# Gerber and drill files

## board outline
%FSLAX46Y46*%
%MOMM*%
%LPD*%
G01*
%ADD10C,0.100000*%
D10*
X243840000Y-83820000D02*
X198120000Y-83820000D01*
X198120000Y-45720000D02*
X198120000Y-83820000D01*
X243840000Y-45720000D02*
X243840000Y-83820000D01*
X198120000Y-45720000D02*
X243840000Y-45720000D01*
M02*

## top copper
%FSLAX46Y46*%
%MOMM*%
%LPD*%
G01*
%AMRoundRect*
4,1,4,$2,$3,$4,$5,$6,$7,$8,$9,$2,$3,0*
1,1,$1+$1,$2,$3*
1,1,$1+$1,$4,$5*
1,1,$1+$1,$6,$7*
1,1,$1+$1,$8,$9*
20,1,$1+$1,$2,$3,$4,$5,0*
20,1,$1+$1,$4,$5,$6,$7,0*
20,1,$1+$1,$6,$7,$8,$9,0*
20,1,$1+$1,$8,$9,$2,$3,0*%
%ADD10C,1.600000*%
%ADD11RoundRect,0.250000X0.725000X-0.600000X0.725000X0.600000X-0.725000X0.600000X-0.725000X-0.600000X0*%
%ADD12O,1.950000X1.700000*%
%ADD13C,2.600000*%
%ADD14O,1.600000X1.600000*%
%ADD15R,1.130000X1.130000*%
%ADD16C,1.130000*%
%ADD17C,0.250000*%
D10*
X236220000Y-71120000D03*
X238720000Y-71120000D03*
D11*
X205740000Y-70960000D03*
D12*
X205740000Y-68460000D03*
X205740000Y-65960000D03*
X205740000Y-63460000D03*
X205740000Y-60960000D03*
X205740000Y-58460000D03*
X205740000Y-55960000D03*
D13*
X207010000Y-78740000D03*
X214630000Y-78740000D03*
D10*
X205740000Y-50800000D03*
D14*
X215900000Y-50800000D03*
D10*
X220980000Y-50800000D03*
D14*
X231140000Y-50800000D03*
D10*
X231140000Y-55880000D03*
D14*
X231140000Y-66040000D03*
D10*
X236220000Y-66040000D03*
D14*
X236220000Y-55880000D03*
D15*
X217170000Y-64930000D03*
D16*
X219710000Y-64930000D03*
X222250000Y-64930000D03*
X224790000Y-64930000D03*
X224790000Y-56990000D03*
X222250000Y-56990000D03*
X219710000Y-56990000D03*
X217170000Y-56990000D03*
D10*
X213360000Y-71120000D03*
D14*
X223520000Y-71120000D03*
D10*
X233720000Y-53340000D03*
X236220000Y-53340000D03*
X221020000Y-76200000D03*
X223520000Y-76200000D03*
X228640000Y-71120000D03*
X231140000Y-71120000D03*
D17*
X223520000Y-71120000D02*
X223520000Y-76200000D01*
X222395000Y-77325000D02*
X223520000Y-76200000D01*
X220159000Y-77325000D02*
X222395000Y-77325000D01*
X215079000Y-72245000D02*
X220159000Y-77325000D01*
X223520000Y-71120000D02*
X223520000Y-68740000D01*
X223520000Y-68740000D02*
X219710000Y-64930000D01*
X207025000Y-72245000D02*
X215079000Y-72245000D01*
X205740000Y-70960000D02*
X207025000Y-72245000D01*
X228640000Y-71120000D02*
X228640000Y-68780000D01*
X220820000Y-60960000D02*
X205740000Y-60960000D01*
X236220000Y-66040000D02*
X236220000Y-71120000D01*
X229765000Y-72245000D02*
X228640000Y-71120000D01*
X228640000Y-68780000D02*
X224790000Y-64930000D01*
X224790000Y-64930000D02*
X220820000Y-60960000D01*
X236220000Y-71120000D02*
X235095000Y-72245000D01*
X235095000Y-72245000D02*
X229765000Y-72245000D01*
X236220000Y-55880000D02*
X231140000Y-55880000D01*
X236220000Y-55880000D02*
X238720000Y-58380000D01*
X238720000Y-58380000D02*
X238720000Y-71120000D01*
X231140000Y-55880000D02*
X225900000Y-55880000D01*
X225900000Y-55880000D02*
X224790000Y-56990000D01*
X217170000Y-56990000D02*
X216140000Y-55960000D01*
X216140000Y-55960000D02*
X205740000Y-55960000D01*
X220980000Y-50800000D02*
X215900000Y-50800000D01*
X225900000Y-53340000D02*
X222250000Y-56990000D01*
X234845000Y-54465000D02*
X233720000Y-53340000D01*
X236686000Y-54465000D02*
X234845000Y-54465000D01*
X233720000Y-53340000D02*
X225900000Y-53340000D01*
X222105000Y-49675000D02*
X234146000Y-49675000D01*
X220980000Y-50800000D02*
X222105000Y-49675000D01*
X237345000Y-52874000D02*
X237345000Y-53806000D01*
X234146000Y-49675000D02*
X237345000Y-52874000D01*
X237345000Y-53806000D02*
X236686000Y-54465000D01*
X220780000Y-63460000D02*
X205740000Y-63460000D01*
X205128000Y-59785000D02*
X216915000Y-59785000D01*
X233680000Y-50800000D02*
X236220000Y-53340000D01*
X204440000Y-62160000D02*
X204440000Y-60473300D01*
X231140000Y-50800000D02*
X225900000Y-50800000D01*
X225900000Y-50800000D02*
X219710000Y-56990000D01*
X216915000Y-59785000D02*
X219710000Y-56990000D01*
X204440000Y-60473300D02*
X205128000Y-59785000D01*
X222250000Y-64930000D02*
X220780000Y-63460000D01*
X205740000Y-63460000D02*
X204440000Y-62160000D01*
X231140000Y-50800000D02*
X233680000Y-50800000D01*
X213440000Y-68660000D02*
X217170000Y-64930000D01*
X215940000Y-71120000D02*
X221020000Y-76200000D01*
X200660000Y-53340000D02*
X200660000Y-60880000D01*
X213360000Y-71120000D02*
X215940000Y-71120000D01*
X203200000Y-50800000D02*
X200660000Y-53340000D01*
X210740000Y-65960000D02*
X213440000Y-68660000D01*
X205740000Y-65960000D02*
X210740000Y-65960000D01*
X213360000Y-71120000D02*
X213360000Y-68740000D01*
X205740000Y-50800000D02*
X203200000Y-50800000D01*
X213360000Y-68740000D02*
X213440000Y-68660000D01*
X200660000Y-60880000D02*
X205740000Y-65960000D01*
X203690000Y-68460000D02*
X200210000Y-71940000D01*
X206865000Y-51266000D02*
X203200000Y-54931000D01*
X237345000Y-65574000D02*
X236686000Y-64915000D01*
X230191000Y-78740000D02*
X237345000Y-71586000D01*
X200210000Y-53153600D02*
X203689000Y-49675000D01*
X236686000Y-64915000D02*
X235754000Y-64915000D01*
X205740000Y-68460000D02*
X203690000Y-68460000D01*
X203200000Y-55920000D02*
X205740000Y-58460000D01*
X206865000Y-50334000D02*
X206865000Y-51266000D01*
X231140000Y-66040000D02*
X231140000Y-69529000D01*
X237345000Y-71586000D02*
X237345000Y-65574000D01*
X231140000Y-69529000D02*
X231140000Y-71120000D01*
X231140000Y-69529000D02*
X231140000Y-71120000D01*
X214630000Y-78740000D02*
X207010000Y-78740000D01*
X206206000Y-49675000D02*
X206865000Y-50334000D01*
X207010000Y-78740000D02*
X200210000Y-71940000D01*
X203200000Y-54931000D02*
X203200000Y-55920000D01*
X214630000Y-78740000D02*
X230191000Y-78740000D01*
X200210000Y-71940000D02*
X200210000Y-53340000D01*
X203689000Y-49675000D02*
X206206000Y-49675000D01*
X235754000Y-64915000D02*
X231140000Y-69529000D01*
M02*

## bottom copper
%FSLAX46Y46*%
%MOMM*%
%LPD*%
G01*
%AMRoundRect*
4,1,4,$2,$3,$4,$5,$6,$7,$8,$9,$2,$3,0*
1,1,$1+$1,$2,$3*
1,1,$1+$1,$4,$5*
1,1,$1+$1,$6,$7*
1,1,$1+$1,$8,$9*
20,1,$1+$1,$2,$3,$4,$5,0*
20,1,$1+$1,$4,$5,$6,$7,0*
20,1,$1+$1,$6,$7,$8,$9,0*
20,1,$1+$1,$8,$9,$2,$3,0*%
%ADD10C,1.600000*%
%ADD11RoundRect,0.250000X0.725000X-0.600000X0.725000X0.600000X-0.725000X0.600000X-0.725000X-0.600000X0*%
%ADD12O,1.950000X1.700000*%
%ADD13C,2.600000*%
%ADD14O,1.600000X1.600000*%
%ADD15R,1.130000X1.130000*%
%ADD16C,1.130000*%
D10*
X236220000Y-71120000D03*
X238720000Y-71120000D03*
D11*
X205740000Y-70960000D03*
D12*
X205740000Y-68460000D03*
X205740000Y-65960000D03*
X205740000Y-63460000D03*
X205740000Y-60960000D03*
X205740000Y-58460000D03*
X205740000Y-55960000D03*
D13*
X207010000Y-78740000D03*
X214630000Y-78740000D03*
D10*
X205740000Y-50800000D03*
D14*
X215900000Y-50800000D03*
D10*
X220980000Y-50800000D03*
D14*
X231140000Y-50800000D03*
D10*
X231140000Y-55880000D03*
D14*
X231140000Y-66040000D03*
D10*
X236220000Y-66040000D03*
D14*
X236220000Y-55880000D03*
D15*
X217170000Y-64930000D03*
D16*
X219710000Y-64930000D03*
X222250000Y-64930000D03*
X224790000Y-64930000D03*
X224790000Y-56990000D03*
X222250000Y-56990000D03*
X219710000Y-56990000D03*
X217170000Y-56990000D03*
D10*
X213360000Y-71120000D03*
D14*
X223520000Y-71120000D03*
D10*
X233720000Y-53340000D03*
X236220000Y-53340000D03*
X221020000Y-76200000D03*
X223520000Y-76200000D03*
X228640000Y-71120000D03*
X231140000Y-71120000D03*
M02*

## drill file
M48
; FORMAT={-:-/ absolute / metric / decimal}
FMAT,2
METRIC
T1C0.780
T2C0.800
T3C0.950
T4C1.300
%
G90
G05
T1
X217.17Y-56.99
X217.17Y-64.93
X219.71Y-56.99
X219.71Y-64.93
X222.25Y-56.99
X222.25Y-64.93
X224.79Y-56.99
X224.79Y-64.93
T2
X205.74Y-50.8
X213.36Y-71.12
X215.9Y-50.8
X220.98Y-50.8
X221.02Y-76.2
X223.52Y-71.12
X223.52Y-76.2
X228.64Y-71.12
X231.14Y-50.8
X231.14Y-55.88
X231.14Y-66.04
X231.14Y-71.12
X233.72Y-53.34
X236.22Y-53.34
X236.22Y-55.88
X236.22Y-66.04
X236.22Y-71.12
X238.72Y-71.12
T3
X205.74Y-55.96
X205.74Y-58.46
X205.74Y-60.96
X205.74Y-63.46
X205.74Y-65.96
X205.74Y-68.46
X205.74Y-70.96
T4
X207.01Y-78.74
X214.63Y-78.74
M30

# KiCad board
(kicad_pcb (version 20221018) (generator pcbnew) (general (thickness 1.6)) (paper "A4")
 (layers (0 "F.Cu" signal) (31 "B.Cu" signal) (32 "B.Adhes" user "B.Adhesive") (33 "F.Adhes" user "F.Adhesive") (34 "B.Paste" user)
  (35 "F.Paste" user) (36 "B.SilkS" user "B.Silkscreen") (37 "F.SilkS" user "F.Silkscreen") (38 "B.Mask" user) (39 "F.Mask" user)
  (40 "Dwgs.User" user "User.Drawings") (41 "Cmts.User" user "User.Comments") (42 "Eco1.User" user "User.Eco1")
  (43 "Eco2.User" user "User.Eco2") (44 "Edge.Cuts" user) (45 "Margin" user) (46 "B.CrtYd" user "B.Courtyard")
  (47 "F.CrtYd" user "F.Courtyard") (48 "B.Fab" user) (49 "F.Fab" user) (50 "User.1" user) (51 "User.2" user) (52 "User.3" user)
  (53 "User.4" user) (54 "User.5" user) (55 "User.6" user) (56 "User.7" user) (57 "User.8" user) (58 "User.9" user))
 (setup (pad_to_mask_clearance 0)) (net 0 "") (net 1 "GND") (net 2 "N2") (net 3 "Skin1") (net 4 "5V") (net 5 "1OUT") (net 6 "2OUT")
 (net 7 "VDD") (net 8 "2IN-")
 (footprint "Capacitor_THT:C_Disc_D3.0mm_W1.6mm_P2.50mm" (layer "F.Cu") (at 236.22 71.12)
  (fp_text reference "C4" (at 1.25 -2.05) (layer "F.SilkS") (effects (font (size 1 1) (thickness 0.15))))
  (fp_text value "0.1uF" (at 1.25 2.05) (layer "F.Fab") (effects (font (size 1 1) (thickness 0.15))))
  (pad "1" thru_hole circle (at 0 0) (size 1.6 1.6) (drill 0.8) (layers "*.Cu" "*.Mask") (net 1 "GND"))
  (pad "2" thru_hole circle (at 2.5 0) (size 1.6 1.6) (drill 0.8) (layers "*.Cu" "*.Mask") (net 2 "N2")))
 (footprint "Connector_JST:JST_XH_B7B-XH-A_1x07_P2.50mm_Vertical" (layer "F.Cu") (at 205.74 70.96 90)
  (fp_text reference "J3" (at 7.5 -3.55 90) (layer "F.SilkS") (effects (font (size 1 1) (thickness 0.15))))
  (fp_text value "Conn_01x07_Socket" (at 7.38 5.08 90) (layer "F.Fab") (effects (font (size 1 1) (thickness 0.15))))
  (pad "1" thru_hole roundrect (at 0 0 90) (size 1.7 1.95) (drill 0.95) (layers "*.Cu" "*.Mask") (roundrect_rratio 0.147059) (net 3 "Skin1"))
  (pad "2" thru_hole oval (at 2.5 0 90) (size 1.7 1.95) (drill 0.95) (layers "*.Cu" "*.Mask") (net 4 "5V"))
  (pad "3" thru_hole oval (at 5 0 90) (size 1.7 1.95) (drill 0.95) (layers "*.Cu" "*.Mask") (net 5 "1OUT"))
  (pad "4" thru_hole oval (at 7.5 0 90) (size 1.7 1.95) (drill 0.95) (layers "*.Cu" "*.Mask") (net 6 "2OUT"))
  (pad "5" thru_hole oval (at 10 0 90) (size 1.7 1.95) (drill 0.95) (layers "*.Cu" "*.Mask") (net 1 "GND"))
  (pad "6" thru_hole oval (at 12.5 0 90) (size 1.7 1.95) (drill 0.95) (layers "*.Cu" "*.Mask") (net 4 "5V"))
  (pad "7" thru_hole oval (at 15 0 90) (size 1.7 1.95) (drill 0.95) (layers "*.Cu" "*.Mask") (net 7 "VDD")))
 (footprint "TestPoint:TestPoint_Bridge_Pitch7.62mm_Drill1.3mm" (layer "F.Cu") (at 207.01 78.74)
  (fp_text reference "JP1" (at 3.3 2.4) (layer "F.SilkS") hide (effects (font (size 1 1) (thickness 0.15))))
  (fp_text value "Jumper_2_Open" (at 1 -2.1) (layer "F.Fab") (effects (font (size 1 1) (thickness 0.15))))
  (pad "1" thru_hole circle (at 0 0) (size 2.6 2.6) (drill 1.3) (layers "*.Cu" "*.Mask") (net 4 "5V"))
  (pad "1" thru_hole circle (at 7.62 0) (size 2.6 2.6) (drill 1.3) (layers "*.Cu" "*.Mask") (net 4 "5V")))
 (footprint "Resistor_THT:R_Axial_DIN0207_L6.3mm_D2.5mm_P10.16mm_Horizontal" (layer "F.Cu") (at 205.74 50.8)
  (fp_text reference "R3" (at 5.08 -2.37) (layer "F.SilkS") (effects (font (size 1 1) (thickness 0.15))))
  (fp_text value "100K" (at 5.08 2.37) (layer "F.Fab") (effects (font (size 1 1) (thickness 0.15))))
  (pad "1" thru_hole circle (at 0 0) (size 1.6 1.6) (drill 0.8) (layers "*.Cu" "*.Mask") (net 5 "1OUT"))
  (pad "2" thru_hole oval (at 10.16 0) (size 1.6 1.6) (drill 0.8) (layers "*.Cu" "*.Mask") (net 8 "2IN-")))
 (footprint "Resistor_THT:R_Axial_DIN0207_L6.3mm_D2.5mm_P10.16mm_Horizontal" (layer "F.Cu") (at 220.98 50.8)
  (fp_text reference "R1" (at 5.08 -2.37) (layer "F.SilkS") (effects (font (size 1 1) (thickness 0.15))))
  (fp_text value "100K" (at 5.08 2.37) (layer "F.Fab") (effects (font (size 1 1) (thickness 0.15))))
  (pad "1" thru_hole circle (at 0 0) (size 1.6 1.6) (drill 0.8) (layers "*.Cu" "*.Mask") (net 8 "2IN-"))
  (pad "2" thru_hole oval (at 10.16 0) (size 1.6 1.6) (drill 0.8) (layers "*.Cu" "*.Mask") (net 6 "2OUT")))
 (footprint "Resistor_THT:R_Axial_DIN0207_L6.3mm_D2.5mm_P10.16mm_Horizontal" (layer "F.Cu") (at 231.14 55.88 -90)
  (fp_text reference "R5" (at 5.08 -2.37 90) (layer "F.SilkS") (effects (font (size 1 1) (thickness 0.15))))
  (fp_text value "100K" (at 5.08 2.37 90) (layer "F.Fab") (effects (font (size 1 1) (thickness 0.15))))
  (pad "1" thru_hole circle (at 0 0 270) (size 1.6 1.6) (drill 0.8) (layers "*.Cu" "*.Mask") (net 2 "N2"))
  (pad "2" thru_hole oval (at 10.16 0 270) (size 1.6 1.6) (drill 0.8) (layers "*.Cu" "*.Mask") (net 4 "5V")))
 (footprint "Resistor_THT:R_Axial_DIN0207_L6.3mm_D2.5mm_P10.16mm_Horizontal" (layer "F.Cu") (at 236.22 66.04 90)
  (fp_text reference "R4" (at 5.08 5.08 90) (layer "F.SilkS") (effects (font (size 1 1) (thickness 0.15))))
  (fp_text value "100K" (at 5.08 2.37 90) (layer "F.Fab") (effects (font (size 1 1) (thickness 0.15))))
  (pad "1" thru_hole circle (at 0 0 90) (size 1.6 1.6) (drill 0.8) (layers "*.Cu" "*.Mask") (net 1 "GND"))
  (pad "2" thru_hole oval (at 10.16 0 90) (size 1.6 1.6) (drill 0.8) (layers "*.Cu" "*.Mask") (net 2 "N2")))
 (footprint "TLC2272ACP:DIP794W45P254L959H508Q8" (layer "F.Cu") (at 220.98 60.96 90)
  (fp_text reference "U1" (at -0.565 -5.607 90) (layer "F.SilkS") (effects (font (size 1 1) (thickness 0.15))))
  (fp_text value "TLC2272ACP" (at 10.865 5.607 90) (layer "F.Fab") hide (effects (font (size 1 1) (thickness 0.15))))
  (pad "1" thru_hole rect (at -3.97 -3.81 90) (size 1.13 1.13) (drill 0.78) (layers "*.Cu" "*.Mask") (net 5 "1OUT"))
  (pad "2" thru_hole circle (at -3.97 -1.27 90) (size 1.13 1.13) (drill 0.78) (layers "*.Cu" "*.Mask") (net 3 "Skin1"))
  (pad "3" thru_hole circle (at -3.97 1.27 90) (size 1.13 1.13) (drill 0.78) (layers "*.Cu" "*.Mask") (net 6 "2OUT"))
  (pad "4" thru_hole circle (at -3.97 3.81 90) (size 1.13 1.13) (drill 0.78) (layers "*.Cu" "*.Mask") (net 1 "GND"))
  (pad "5" thru_hole circle (at 3.97 3.81 90) (size 1.13 1.13) (drill 0.78) (layers "*.Cu" "*.Mask") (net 2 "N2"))
  (pad "6" thru_hole circle (at 3.97 1.27 90) (size 1.13 1.13) (drill 0.78) (layers "*.Cu" "*.Mask") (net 8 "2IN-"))
  (pad "7" thru_hole circle (at 3.97 -1.27 90) (size 1.13 1.13) (drill 0.78) (layers "*.Cu" "*.Mask") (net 6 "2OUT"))
  (pad "8" thru_hole circle (at 3.97 -3.81 90) (size 1.13 1.13) (drill 0.78) (layers "*.Cu" "*.Mask") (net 7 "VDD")))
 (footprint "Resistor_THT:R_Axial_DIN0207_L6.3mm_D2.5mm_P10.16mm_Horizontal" (layer "F.Cu") (at 213.36 71.12)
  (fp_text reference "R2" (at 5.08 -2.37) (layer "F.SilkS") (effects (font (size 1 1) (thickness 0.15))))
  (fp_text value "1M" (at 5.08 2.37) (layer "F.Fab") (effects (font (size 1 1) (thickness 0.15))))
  (pad "1" thru_hole circle (at 0 0) (size 1.6 1.6) (drill 0.8) (layers "*.Cu" "*.Mask") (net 5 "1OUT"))
  (pad "2" thru_hole oval (at 10.16 0) (size 1.6 1.6) (drill 0.8) (layers "*.Cu" "*.Mask") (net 3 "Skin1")))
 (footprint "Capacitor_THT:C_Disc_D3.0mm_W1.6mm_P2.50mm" (layer "F.Cu") (at 233.72 53.34)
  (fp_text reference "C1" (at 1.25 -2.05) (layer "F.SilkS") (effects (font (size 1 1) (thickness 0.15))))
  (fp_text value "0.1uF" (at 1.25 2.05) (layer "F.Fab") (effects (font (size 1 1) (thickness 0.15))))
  (pad "1" thru_hole circle (at 0 0) (size 1.6 1.6) (drill 0.8) (layers "*.Cu" "*.Mask") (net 8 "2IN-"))
  (pad "2" thru_hole circle (at 2.5 0) (size 1.6 1.6) (drill 0.8) (layers "*.Cu" "*.Mask") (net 6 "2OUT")))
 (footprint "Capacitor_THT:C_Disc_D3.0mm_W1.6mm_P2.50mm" (layer "F.Cu") (at 221.02 76.2)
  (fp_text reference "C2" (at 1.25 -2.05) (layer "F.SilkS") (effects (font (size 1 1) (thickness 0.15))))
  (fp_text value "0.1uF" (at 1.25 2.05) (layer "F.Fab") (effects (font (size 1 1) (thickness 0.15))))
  (pad "1" thru_hole circle (at 0 0) (size 1.6 1.6) (drill 0.8) (layers "*.Cu" "*.Mask") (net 5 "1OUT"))
  (pad "2" thru_hole circle (at 2.5 0) (size 1.6 1.6) (drill 0.8) (layers "*.Cu" "*.Mask") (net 3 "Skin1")))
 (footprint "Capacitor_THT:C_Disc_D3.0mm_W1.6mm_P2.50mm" (layer "F.Cu") (at 228.64 71.12)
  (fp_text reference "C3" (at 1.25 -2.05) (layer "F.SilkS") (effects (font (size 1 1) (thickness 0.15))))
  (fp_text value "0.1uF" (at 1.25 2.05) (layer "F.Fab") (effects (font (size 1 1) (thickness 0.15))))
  (pad "1" thru_hole circle (at 0 0) (size 1.6 1.6) (drill 0.8) (layers "*.Cu" "*.Mask") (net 1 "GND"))
  (pad "2" thru_hole circle (at 2.5 0) (size 1.6 1.6) (drill 0.8) (layers "*.Cu" "*.Mask") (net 4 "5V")))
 (gr_line (start 243.84 83.82) (end 198.12 83.82) (stroke (width 0.1) (type default)) (layer "Edge.Cuts"))
 (gr_line (start 198.12 45.72) (end 198.12 83.82) (stroke (width 0.1) (type default)) (layer "Edge.Cuts"))
 (gr_line (start 243.84 45.72) (end 243.84 83.82) (stroke (width 0.1) (type default)) (layer "Edge.Cuts"))
 (gr_line (start 198.12 45.72) (end 243.84 45.72) (stroke (width 0.1) (type default)) (layer "Edge.Cuts"))
 (segment (start 223.52 71.12) (end 223.52 76.2) (width 0.25) (layer "F.Cu") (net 3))
 (segment (start 222.395 77.325) (end 223.52 76.2) (width 0.25) (layer "F.Cu") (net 3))
 (segment (start 220.159 77.325) (end 222.395 77.325) (width 0.25) (layer "F.Cu") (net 3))
 (segment (start 215.079 72.245) (end 220.159 77.325) (width 0.25) (layer "F.Cu") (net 3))
 (segment (start 223.52 71.12) (end 223.52 68.74) (width 0.25) (layer "F.Cu") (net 3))
 (segment (start 223.52 68.74) (end 219.71 64.93) (width 0.25) (layer "F.Cu") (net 3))
 (segment (start 207.025 72.245) (end 215.079 72.245) (width 0.25) (layer "F.Cu") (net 3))
 (segment (start 205.74 70.96) (end 207.025 72.245) (width 0.25) (layer "F.Cu") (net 3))
 (segment (start 228.64 71.12) (end 228.64 68.78) (width 0.25) (layer "F.Cu") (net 1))
 (segment (start 220.82 60.96) (end 205.74 60.96) (width 0.25) (layer "F.Cu") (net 1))
 (segment (start 236.22 66.04) (end 236.22 71.12) (width 0.25) (layer "F.Cu") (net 1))
 (segment (start 229.765 72.245) (end 228.64 71.12) (width 0.25) (layer "F.Cu") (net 1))
 (segment (start 228.64 68.78) (end 224.79 64.93) (width 0.25) (layer "F.Cu") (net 1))
 (segment (start 224.79 64.93) (end 220.82 60.96) (width 0.25) (layer "F.Cu") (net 1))
 (segment (start 236.22 71.12) (end 235.095 72.245) (width 0.25) (layer "F.Cu") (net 1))
 (segment (start 235.095 72.245) (end 229.765 72.245) (width 0.25) (layer "F.Cu") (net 1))
 (segment (start 236.22 55.88) (end 231.14 55.88) (width 0.25) (layer "F.Cu") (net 2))
 (segment (start 236.22 55.88) (end 238.72 58.38) (width 0.25) (layer "F.Cu") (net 2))
 (segment (start 238.72 58.38) (end 238.72 71.12) (width 0.25) (layer "F.Cu") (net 2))
 (segment (start 231.14 55.88) (end 225.9 55.88) (width 0.25) (layer "F.Cu") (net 2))
 (segment (start 225.9 55.88) (end 224.79 56.99) (width 0.25) (layer "F.Cu") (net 2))
 (segment (start 217.17 56.99) (end 216.14 55.96) (width 0.25) (layer "F.Cu") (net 7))
 (segment (start 216.14 55.96) (end 205.74 55.96) (width 0.25) (layer "F.Cu") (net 7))
 (segment (start 220.98 50.8) (end 215.9 50.8) (width 0.25) (layer "F.Cu") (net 8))
 (segment (start 225.9 53.34) (end 222.25 56.99) (width 0.25) (layer "F.Cu") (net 8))
 (segment (start 234.845 54.465) (end 233.72 53.34) (width 0.25) (layer "F.Cu") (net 8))
 (segment (start 236.686 54.465) (end 234.845 54.465) (width 0.25) (layer "F.Cu") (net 8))
 (segment (start 233.72 53.34) (end 225.9 53.34) (width 0.25) (layer "F.Cu") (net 8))
 (segment (start 222.105 49.675) (end 234.146 49.675) (width 0.25) (layer "F.Cu") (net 8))
 (segment (start 220.98 50.8) (end 222.105 49.675) (width 0.25) (layer "F.Cu") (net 8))
 (segment (start 237.345 52.874) (end 237.345 53.806) (width 0.25) (layer "F.Cu") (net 8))
 (segment (start 234.146 49.675) (end 237.345 52.874) (width 0.25) (layer "F.Cu") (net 8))
 (segment (start 237.345 53.806) (end 236.686 54.465) (width 0.25) (layer "F.Cu") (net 8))
 (segment (start 220.78 63.46) (end 205.74 63.46) (width 0.25) (layer "F.Cu") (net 6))
 (segment (start 205.128 59.785) (end 216.915 59.785) (width 0.25) (layer "F.Cu") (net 6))
 (segment (start 233.68 50.8) (end 236.22 53.34) (width 0.25) (layer "F.Cu") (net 6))
 (segment (start 204.44 62.16) (end 204.44 60.4733) (width 0.25) (layer "F.Cu") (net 6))
 (segment (start 231.14 50.8) (end 225.9 50.8) (width 0.25) (layer "F.Cu") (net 6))
 (segment (start 225.9 50.8) (end 219.71 56.99) (width 0.25) (layer "F.Cu") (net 6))
 (segment (start 216.915 59.785) (end 219.71 56.99) (width 0.25) (layer "F.Cu") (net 6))
 (segment (start 204.44 60.4733) (end 205.128 59.785) (width 0.25) (layer "F.Cu") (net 6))
 (segment (start 222.25 64.93) (end 220.78 63.46) (width 0.25) (layer "F.Cu") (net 6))
 (segment (start 205.74 63.46) (end 204.44 62.16) (width 0.25) (layer "F.Cu") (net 6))
 (segment (start 231.14 50.8) (end 233.68 50.8) (width 0.25) (layer "F.Cu") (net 6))
 (segment (start 213.44 68.66) (end 217.17 64.93) (width 0.25) (layer "F.Cu") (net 5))
 (segment (start 215.94 71.12) (end 221.02 76.2) (width 0.25) (layer "F.Cu") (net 5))
 (segment (start 200.66 53.34) (end 200.66 60.88) (width 0.25) (layer "F.Cu") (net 5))
 (segment (start 213.36 71.12) (end 215.94 71.12) (width 0.25) (layer "F.Cu") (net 5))
 (segment (start 203.2 50.8) (end 200.66 53.34) (width 0.25) (layer "F.Cu") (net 5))
 (segment (start 210.74 65.96) (end 213.44 68.66) (width 0.25) (layer "F.Cu") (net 5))
 (segment (start 205.74 65.96) (end 210.74 65.96) (width 0.25) (layer "F.Cu") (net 5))
 (segment (start 213.36 71.12) (end 213.36 68.74) (width 0.25) (layer "F.Cu") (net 5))
 (segment (start 205.74 50.8) (end 203.2 50.8) (width 0.25) (layer "F.Cu") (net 5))
 (segment (start 213.36 68.74) (end 213.44 68.66) (width 0.25) (layer "F.Cu") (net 5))
 (segment (start 200.66 60.88) (end 205.74 65.96) (width 0.25) (layer "F.Cu") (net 5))
 (segment (start 203.69 68.46) (end 200.21 71.94) (width 0.25) (layer "F.Cu") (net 4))
 (segment (start 206.865 51.266) (end 203.2 54.931) (width 0.25) (layer "F.Cu") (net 4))
 (segment (start 237.345 65.574) (end 236.686 64.915) (width 0.25) (layer "F.Cu") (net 4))
 (segment (start 230.191 78.74) (end 237.345 71.586) (width 0.25) (layer "F.Cu") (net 4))
 (segment (start 200.21 53.1536) (end 203.689 49.675) (width 0.25) (layer "F.Cu") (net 4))
 (segment (start 236.686 64.915) (end 235.754 64.915) (width 0.25) (layer "F.Cu") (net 4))
 (segment (start 205.74 68.46) (end 203.69 68.46) (width 0.25) (layer "F.Cu") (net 4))
 (segment (start 203.2 55.92) (end 205.74 58.46) (width 0.25) (layer "F.Cu") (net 4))
 (segment (start 206.865 50.334) (end 206.865 51.266) (width 0.25) (layer "F.Cu") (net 4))
 (segment (start 231.14 66.04) (end 231.14 69.529) (width 0.25) (layer "F.Cu") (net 4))
 (segment (start 237.345 71.586) (end 237.345 65.574) (width 0.25) (layer "F.Cu") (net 4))
 (segment (start 231.14 69.529) (end 231.14 71.12) (width 0.25) (layer "F.Cu") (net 4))
 (segment (start 231.14 69.529) (end 231.14 71.12) (width 0.25) (layer "F.Cu") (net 4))
 (segment (start 214.63 78.74) (end 207.01 78.74) (width 0.25) (layer "F.Cu") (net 4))
 (segment (start 206.206 49.675) (end 206.865 50.334) (width 0.25) (layer "F.Cu") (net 4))
 (segment (start 207.01 78.74) (end 200.21 71.94) (width 0.25) (layer "F.Cu") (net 4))
 (segment (start 203.2 54.931) (end 203.2 55.92) (width 0.25) (layer "F.Cu") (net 4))
 (segment (start 214.63 78.74) (end 230.191 78.74) (width 0.25) (layer "F.Cu") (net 4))
 (segment (start 200.21 71.94) (end 200.21 53.34) (width 0.25) (layer "F.Cu") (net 4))
 (segment (start 203.689 49.675) (end 206.206 49.675) (width 0.25) (layer "F.Cu") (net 4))
 (segment (start 235.754 64.915) (end 231.14 69.529) (width 0.25) (layer "F.Cu") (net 4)))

